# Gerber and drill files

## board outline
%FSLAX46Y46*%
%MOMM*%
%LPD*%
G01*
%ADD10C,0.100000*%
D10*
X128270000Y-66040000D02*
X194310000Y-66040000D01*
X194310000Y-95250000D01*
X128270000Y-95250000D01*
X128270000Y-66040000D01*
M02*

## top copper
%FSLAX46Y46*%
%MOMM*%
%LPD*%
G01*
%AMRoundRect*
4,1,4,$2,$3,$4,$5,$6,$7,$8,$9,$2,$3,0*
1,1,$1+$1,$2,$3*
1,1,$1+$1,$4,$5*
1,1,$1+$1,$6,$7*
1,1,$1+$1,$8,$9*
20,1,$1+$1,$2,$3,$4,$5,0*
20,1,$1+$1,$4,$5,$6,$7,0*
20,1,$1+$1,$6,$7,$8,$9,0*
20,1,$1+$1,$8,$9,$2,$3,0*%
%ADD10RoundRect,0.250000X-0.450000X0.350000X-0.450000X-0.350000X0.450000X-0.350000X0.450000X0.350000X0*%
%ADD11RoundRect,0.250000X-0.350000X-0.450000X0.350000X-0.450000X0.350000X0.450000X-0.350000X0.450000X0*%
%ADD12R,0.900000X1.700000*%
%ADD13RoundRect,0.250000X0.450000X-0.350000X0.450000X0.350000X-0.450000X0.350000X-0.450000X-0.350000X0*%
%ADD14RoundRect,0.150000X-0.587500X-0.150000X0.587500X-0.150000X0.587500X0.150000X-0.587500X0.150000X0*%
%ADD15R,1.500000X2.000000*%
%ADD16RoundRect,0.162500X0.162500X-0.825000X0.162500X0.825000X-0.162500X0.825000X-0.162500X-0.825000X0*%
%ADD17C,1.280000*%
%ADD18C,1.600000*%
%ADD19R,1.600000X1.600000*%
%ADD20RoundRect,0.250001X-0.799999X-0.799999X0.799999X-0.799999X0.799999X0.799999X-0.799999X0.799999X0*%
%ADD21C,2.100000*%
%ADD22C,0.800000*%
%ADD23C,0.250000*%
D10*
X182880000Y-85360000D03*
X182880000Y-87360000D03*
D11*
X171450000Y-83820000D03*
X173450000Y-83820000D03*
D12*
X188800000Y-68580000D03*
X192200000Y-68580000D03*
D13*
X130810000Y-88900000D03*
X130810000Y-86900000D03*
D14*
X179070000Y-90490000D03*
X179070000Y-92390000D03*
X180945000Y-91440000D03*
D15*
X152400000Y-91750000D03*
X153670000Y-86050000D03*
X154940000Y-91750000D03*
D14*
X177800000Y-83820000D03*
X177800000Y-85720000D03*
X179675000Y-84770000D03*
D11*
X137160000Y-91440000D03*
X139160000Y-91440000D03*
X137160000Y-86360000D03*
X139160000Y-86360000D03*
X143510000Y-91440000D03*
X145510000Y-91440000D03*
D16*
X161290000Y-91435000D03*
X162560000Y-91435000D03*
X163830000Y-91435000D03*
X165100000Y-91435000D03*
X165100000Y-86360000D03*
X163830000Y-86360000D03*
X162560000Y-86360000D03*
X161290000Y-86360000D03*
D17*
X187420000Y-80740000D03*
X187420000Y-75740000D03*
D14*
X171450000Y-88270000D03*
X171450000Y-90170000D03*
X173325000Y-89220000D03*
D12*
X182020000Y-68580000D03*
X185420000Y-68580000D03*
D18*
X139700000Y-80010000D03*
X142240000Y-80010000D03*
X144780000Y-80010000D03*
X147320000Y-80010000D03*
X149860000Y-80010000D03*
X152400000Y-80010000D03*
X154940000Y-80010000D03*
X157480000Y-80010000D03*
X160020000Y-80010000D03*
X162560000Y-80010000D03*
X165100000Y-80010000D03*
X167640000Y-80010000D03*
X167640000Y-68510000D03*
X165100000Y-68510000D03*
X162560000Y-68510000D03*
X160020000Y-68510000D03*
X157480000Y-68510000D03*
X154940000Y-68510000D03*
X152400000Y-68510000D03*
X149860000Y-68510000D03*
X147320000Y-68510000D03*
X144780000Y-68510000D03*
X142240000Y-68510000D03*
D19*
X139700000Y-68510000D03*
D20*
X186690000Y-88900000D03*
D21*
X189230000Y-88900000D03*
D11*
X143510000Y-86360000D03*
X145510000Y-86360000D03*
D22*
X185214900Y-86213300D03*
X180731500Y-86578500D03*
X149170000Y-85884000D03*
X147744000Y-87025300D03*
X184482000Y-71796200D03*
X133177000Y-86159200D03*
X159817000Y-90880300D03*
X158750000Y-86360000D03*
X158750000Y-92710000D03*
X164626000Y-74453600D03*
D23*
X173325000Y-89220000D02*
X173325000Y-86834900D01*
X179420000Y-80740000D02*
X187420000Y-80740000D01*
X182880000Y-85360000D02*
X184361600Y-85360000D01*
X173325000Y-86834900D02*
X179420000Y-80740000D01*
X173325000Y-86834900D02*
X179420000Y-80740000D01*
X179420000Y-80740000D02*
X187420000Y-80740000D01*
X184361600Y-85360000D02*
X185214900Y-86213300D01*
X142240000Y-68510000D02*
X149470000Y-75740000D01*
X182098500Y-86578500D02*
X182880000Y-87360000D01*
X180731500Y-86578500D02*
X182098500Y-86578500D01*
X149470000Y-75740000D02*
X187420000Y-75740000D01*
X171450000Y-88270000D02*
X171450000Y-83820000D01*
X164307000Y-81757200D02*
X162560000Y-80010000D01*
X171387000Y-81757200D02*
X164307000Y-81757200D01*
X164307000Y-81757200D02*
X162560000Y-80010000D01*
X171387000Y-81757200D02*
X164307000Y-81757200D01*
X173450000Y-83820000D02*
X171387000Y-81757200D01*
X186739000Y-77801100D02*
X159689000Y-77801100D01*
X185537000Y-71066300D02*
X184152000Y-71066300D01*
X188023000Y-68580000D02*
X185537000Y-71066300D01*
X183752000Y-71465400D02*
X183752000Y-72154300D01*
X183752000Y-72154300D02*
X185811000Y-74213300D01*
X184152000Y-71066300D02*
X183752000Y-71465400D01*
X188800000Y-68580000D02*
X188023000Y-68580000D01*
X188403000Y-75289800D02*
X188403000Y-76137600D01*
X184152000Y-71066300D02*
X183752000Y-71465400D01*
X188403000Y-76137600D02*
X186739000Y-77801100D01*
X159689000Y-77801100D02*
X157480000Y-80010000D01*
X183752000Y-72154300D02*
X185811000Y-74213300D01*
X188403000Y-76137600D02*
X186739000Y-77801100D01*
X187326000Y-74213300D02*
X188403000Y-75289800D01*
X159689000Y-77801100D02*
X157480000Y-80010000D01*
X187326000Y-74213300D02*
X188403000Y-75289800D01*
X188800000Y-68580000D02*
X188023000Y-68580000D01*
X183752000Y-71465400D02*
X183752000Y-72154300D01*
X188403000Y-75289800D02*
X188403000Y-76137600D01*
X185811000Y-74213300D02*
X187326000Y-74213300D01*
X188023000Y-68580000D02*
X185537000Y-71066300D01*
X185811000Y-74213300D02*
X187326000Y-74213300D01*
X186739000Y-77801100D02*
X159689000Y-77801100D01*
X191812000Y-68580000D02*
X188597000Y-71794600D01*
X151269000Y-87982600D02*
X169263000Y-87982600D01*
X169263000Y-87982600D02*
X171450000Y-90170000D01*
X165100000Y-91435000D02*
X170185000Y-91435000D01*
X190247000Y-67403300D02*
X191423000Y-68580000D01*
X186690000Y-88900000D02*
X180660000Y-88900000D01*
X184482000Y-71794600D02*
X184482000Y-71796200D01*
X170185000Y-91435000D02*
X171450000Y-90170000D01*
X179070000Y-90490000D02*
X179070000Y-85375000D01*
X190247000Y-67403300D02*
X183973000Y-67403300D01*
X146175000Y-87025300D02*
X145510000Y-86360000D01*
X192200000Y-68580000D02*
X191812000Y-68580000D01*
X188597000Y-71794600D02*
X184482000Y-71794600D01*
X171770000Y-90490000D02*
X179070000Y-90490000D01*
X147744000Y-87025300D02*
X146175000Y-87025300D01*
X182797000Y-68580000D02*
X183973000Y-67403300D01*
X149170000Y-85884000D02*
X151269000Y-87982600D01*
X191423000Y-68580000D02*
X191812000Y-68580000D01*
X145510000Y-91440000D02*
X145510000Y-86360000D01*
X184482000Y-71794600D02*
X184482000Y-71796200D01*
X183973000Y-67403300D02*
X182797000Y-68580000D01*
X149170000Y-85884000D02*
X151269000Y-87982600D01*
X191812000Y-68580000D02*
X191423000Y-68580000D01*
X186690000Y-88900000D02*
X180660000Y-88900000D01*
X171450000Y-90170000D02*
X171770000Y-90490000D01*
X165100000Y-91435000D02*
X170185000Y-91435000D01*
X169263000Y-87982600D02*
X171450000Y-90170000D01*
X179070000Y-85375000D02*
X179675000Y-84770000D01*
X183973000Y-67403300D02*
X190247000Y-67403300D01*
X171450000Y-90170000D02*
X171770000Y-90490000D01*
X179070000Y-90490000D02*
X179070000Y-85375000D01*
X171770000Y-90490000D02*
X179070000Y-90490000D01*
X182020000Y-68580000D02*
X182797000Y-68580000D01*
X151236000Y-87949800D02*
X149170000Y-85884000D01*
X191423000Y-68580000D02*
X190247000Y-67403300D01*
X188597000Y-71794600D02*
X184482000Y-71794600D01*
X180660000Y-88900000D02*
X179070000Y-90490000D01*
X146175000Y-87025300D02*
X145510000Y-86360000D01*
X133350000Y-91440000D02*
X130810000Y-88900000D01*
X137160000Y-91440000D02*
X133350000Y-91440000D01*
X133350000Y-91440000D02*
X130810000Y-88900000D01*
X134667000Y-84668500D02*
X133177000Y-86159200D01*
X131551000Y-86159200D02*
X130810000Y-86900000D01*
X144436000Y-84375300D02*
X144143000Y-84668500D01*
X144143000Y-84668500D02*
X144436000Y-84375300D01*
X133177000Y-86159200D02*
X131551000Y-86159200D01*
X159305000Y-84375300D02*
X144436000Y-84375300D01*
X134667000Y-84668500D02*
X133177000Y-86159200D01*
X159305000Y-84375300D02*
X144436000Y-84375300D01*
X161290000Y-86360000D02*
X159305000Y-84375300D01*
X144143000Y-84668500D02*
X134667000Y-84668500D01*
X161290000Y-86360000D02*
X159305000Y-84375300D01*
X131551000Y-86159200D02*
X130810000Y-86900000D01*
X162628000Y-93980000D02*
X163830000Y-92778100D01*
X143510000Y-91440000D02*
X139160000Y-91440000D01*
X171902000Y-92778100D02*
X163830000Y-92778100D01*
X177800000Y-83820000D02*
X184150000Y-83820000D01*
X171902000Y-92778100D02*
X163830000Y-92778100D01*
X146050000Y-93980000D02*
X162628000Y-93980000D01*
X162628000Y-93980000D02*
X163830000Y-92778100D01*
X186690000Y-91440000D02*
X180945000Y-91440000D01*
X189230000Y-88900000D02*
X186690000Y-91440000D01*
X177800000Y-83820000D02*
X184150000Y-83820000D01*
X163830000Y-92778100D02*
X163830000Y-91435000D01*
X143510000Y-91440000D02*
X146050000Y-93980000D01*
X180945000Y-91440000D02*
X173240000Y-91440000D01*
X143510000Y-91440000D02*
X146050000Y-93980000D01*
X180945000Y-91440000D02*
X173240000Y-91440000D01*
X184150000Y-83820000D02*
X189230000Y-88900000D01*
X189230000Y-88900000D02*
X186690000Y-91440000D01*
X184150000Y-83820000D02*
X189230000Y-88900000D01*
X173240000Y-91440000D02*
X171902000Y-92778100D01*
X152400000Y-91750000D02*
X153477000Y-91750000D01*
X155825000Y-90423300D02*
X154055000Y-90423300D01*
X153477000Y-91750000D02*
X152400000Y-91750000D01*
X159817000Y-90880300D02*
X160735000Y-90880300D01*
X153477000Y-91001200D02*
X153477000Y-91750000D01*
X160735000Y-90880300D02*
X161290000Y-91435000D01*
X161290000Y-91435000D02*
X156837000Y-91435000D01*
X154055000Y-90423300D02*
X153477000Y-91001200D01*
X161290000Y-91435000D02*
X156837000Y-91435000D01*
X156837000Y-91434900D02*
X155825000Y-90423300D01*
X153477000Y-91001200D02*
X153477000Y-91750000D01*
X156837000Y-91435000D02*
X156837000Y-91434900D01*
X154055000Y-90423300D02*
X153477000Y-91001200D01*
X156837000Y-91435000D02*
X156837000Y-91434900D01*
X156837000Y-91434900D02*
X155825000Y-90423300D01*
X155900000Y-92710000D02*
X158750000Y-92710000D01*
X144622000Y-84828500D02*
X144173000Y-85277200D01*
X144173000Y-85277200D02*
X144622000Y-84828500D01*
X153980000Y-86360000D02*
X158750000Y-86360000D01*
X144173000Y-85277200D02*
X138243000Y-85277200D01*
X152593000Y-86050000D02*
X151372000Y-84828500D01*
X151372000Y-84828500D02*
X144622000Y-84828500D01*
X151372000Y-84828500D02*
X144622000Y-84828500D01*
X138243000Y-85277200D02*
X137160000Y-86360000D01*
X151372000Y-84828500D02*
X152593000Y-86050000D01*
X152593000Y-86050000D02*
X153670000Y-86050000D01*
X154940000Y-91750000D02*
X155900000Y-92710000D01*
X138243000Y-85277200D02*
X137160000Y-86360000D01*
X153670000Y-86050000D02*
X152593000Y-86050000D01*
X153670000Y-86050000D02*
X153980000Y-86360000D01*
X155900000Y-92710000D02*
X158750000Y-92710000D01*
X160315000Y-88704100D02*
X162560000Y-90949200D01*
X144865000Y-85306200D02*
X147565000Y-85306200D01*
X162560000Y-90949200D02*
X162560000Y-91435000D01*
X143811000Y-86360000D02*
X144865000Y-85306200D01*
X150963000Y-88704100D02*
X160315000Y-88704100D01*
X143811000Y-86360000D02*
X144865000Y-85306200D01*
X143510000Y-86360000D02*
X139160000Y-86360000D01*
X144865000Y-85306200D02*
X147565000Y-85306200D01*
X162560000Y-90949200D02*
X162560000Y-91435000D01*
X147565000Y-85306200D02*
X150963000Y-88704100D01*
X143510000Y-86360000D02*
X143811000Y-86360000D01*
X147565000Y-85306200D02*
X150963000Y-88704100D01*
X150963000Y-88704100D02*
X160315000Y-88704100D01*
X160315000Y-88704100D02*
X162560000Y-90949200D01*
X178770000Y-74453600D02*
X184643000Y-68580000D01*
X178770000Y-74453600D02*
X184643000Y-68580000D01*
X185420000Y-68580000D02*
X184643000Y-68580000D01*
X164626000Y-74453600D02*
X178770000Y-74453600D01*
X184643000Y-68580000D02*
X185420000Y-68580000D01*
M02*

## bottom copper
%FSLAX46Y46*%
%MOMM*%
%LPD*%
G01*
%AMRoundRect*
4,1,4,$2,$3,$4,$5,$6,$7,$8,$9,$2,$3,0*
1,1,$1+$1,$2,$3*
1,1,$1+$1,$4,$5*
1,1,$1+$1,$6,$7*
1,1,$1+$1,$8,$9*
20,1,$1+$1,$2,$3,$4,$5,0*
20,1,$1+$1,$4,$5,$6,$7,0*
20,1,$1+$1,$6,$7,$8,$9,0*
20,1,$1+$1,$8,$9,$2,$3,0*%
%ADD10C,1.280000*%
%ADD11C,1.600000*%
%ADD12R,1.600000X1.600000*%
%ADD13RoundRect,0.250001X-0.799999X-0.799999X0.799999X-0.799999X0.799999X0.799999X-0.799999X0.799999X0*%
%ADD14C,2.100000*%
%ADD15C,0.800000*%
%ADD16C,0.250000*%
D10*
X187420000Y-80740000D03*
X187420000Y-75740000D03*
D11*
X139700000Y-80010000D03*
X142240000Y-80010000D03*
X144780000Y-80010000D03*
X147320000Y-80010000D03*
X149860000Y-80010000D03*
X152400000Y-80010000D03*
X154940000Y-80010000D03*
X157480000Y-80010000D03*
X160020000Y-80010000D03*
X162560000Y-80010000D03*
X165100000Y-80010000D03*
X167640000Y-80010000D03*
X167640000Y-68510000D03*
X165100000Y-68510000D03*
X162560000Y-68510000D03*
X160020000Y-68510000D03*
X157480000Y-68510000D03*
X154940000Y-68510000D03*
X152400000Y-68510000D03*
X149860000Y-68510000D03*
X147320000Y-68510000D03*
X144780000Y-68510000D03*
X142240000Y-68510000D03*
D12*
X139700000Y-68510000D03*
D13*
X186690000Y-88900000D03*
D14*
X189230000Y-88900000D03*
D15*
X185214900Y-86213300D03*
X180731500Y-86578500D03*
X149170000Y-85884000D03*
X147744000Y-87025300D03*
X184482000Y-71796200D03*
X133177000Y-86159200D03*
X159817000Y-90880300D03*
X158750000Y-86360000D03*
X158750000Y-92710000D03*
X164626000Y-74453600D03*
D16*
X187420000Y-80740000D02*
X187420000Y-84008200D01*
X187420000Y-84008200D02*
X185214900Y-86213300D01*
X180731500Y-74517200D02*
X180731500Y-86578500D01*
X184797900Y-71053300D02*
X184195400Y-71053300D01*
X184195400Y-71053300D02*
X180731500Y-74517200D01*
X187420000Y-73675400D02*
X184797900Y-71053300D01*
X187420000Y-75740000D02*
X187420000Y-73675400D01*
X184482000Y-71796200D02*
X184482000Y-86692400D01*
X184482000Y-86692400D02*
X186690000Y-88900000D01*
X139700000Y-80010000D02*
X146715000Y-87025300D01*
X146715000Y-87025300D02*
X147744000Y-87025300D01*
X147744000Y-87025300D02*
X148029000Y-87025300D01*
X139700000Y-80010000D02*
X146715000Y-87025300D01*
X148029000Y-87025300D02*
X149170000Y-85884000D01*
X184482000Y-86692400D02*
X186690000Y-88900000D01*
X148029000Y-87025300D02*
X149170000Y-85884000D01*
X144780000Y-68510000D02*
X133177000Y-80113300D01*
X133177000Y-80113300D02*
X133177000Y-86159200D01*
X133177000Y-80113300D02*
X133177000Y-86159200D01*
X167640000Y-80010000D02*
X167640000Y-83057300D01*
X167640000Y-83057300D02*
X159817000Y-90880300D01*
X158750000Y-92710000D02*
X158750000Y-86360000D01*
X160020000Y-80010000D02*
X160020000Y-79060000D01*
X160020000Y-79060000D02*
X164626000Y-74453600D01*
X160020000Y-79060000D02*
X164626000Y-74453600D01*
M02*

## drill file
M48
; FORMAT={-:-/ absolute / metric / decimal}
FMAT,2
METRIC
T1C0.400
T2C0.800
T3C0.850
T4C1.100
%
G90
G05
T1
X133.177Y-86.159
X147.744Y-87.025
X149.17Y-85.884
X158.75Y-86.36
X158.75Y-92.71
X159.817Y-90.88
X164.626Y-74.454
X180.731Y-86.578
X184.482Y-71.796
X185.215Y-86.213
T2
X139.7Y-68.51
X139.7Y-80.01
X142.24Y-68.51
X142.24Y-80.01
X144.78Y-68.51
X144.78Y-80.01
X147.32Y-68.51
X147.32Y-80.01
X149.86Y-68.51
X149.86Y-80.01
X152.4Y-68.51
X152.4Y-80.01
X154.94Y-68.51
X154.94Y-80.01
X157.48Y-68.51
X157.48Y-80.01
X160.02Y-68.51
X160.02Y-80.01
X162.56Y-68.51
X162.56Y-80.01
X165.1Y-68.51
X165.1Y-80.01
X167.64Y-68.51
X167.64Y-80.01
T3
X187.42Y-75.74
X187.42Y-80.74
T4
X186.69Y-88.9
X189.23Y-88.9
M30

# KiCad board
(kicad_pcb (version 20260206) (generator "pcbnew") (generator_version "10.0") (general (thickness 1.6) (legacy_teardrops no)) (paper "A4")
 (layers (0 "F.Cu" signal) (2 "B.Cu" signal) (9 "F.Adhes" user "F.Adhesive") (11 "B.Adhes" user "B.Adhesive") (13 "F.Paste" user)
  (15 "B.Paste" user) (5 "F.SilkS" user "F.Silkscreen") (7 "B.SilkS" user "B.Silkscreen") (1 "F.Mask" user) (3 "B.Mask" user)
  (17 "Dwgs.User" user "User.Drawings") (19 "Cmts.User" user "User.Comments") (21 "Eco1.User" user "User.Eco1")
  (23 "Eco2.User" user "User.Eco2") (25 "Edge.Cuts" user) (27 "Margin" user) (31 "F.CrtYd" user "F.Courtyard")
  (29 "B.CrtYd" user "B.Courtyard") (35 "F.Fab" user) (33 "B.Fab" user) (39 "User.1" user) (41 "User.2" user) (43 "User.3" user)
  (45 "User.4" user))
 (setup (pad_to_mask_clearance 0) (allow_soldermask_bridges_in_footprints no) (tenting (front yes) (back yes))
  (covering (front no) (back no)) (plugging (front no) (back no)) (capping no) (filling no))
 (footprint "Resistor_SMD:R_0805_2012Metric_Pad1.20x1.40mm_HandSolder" (layer "F.Cu") (at 182.88 86.36 -90)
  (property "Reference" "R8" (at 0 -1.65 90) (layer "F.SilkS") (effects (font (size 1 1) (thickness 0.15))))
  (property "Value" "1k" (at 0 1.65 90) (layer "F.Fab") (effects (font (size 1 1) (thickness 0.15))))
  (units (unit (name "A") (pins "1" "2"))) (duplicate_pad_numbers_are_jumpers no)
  (pad "1" smd roundrect (at -1 0 270) (size 1.2 1.4) (layers "F.Cu" "F.Mask" "F.Paste") (roundrect_rratio 0.208333) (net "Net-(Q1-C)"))
  (pad "2" smd roundrect (at 1 0 270) (size 1.2 1.4) (layers "F.Cu" "F.Mask" "F.Paste") (roundrect_rratio 0.208333) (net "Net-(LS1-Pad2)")))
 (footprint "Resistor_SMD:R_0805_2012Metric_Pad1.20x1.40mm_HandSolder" (layer "F.Cu") (at 172.45 83.82)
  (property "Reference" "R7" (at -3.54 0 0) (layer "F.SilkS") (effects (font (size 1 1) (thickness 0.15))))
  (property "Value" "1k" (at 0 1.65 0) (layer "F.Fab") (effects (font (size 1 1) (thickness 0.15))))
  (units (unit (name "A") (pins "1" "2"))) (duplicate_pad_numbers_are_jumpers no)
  (pad "1" smd roundrect (at -1 0) (size 1.2 1.4) (layers "F.Cu" "F.Mask" "F.Paste") (roundrect_rratio 0.208333) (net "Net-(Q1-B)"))
  (pad "2" smd roundrect (at 1 0) (size 1.2 1.4) (layers "F.Cu" "F.Mask" "F.Paste") (roundrect_rratio 0.208333) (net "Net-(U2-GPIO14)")))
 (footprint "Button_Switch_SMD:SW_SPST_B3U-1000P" (layer "F.Cu") (at 190.5 68.58)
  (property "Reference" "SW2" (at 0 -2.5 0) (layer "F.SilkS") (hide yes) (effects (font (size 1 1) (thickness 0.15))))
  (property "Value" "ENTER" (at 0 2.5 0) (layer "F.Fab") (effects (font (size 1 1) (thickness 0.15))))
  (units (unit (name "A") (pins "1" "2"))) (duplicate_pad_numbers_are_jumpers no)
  (pad "1" smd rect (at -1.7 0) (size 0.9 1.7) (layers "F.Cu" "F.Mask" "F.Paste") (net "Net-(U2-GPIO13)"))
  (pad "2" smd rect (at 1.7 0) (size 0.9 1.7) (layers "F.Cu" "F.Mask" "F.Paste") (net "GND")))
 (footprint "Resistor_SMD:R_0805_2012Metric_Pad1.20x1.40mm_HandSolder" (layer "F.Cu") (at 130.81 87.9 90)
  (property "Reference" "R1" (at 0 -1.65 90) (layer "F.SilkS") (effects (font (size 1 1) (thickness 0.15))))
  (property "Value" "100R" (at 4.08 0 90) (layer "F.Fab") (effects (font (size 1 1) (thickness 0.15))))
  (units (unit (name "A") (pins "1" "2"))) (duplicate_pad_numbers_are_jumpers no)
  (pad "1" smd roundrect (at -1 0 90) (size 1.2 1.4) (layers "F.Cu" "F.Mask" "F.Paste") (roundrect_rratio 0.208333) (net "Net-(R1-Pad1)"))
  (pad "2" smd roundrect (at 1 0 90) (size 1.2 1.4) (layers "F.Cu" "F.Mask" "F.Paste") (roundrect_rratio 0.208333) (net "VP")))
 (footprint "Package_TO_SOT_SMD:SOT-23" (layer "F.Cu") (at 180.0075 91.44)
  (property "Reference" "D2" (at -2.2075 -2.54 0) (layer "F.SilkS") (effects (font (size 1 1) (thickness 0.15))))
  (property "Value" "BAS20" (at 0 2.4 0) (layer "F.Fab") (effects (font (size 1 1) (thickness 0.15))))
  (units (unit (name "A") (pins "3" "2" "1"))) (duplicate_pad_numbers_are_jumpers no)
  (pad "1" smd roundrect (at -0.9375 -0.95) (size 1.475 0.6) (layers "F.Cu" "F.Mask" "F.Paste") (roundrect_rratio 0.25) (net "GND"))
  (pad "2" smd roundrect (at -0.9375 0.95) (size 1.475 0.6) (layers "F.Cu" "F.Mask" "F.Paste") (roundrect_rratio 0.25)
   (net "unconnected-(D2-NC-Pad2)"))
  (pad "3" smd roundrect (at 0.9375 0) (size 1.475 0.6) (layers "F.Cu" "F.Mask" "F.Paste") (roundrect_rratio 0.25) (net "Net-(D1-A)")))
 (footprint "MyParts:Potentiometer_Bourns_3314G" (layer "F.Cu") (at 153.67 88.9)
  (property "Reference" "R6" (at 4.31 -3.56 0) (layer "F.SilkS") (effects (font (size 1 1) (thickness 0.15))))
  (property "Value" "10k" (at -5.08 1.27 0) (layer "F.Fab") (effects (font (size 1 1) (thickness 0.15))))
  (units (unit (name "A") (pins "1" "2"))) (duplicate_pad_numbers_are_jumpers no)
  (pad "1" smd rect (at -1.27 2.85) (size 1.5 2) (layers "F.Cu" "F.Mask" "F.Paste") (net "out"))
  (pad "2" smd rect (at 0 -2.85) (size 1.5 2) (layers "F.Cu" "F.Mask" "F.Paste") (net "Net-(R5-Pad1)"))
  (pad "3" smd rect (at 1.27 2.85) (size 1.5 2) (layers "F.Cu" "F.Mask" "F.Paste")))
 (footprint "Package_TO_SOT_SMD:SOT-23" (layer "F.Cu") (at 178.7375 84.77)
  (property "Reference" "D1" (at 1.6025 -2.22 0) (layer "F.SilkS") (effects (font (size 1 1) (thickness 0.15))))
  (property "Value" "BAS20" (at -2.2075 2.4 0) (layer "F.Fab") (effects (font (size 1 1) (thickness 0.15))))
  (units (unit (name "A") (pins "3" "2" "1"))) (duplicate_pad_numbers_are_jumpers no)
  (pad "1" smd roundrect (at -0.9375 -0.95) (size 1.475 0.6) (layers "F.Cu" "F.Mask" "F.Paste") (roundrect_rratio 0.25) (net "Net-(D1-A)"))
  (pad "2" smd roundrect (at -0.9375 0.95) (size 1.475 0.6) (layers "F.Cu" "F.Mask" "F.Paste") (roundrect_rratio 0.25)
   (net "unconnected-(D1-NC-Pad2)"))
  (pad "3" smd roundrect (at 0.9375 0) (size 1.475 0.6) (layers "F.Cu" "F.Mask" "F.Paste") (roundrect_rratio 0.25) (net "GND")))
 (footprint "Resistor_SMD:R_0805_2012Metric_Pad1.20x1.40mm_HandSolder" (layer "F.Cu") (at 138.16 91.44)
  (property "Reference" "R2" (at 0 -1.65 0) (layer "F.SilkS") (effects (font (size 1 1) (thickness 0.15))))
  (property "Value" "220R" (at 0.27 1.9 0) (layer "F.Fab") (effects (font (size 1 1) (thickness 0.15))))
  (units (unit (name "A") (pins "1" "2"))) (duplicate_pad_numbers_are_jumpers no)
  (pad "1" smd roundrect (at -1 0) (size 1.2 1.4) (layers "F.Cu" "F.Mask" "F.Paste") (roundrect_rratio 0.208333) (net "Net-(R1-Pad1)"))
  (pad "2" smd roundrect (at 1 0) (size 1.2 1.4) (layers "F.Cu" "F.Mask" "F.Paste") (roundrect_rratio 0.208333) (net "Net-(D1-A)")))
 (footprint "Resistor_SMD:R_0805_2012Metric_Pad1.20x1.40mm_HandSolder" (layer "F.Cu") (at 138.16 86.36)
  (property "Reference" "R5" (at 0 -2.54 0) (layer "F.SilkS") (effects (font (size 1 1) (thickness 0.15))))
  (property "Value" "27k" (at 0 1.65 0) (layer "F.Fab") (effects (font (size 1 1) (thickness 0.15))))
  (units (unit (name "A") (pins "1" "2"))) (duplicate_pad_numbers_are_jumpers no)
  (pad "1" smd roundrect (at -1 0) (size 1.2 1.4) (layers "F.Cu" "F.Mask" "F.Paste") (roundrect_rratio 0.208333) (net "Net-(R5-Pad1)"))
  (pad "2" smd roundrect (at 1 0) (size 1.2 1.4) (layers "F.Cu" "F.Mask" "F.Paste") (roundrect_rratio 0.208333) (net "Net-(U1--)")))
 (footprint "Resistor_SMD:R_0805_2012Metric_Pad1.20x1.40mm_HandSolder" (layer "F.Cu") (at 144.51 91.44)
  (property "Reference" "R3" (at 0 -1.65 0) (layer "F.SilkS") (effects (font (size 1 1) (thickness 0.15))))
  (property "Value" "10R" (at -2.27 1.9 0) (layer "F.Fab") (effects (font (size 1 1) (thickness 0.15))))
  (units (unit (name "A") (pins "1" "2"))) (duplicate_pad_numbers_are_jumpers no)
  (pad "1" smd roundrect (at -1 0) (size 1.2 1.4) (layers "F.Cu" "F.Mask" "F.Paste") (roundrect_rratio 0.208333) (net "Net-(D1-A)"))
  (pad "2" smd roundrect (at 1 0) (size 1.2 1.4) (layers "F.Cu" "F.Mask" "F.Paste") (roundrect_rratio 0.208333) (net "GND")))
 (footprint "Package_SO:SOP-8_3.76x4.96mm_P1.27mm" (layer "F.Cu") (at 163.195 88.8975 90)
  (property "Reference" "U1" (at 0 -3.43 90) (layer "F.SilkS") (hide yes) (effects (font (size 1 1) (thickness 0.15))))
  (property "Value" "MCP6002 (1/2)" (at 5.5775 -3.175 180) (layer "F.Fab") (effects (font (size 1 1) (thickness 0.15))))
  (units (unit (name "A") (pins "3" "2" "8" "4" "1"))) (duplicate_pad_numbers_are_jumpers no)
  (pad "1" smd roundrect (at -2.5375 -1.905 90) (size 1.975 0.65) (layers "F.Cu" "F.Mask" "F.Paste") (roundrect_rratio 0.25) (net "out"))
  (pad "2" smd roundrect (at -2.5375 -0.635 90) (size 1.975 0.65) (layers "F.Cu" "F.Mask" "F.Paste") (roundrect_rratio 0.25)
   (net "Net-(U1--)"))
  (pad "3" smd roundrect (at -2.5375 0.635 90) (size 1.975 0.65) (layers "F.Cu" "F.Mask" "F.Paste") (roundrect_rratio 0.25)
   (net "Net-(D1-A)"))
  (pad "4" smd roundrect (at -2.5375 1.905 90) (size 1.975 0.65) (layers "F.Cu" "F.Mask" "F.Paste") (roundrect_rratio 0.25) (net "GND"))
  (pad "5" smd roundrect (at 2.5375 1.905 90) (size 1.975 0.65) (layers "F.Cu" "F.Mask" "F.Paste") (roundrect_rratio 0.25))
  (pad "6" smd roundrect (at 2.5375 0.635 90) (size 1.975 0.65) (layers "F.Cu" "F.Mask" "F.Paste") (roundrect_rratio 0.25))
  (pad "7" smd roundrect (at 2.5375 -0.635 90) (size 1.975 0.65) (layers "F.Cu" "F.Mask" "F.Paste") (roundrect_rratio 0.25))
  (pad "8" smd roundrect (at 2.5375 -1.905 90) (size 1.975 0.65) (layers "F.Cu" "F.Mask" "F.Paste") (roundrect_rratio 0.25) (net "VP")))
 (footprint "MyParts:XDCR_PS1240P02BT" (layer "F.Cu") (at 187.42 78.24 90)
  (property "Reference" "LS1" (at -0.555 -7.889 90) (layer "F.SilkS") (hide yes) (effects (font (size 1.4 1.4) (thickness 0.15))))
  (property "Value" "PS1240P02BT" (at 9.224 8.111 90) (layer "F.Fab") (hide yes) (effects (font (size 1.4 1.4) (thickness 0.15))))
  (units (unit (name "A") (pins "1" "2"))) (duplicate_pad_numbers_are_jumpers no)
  (pad "1" thru_hole circle (at -2.5 0 90) (size 1.28 1.28) (drill 0.85) (layers "*.Cu" "*.Mask") (remove_unused_layers no)
   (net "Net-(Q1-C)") (solder_mask_margin 0.102))
  (pad "2" thru_hole circle (at 2.5 0 90) (size 1.28 1.28) (drill 0.85) (layers "*.Cu" "*.Mask") (remove_unused_layers no)
   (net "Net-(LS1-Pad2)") (solder_mask_margin 0.102)))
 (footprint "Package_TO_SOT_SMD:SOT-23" (layer "F.Cu") (at 172.3875 89.22)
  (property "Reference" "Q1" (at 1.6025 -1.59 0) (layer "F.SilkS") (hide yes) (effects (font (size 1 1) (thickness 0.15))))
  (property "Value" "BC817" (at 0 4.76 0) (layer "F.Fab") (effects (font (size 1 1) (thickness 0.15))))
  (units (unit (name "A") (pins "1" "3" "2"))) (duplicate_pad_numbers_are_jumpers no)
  (pad "1" smd roundrect (at -0.9375 -0.95) (size 1.475 0.6) (layers "F.Cu" "F.Mask" "F.Paste") (roundrect_rratio 0.25) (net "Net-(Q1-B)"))
  (pad "2" smd roundrect (at -0.9375 0.95) (size 1.475 0.6) (layers "F.Cu" "F.Mask" "F.Paste") (roundrect_rratio 0.25) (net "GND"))
  (pad "3" smd roundrect (at 0.9375 0) (size 1.475 0.6) (layers "F.Cu" "F.Mask" "F.Paste") (roundrect_rratio 0.25) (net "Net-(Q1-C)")))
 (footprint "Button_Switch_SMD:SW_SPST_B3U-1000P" (layer "F.Cu") (at 183.72 68.58)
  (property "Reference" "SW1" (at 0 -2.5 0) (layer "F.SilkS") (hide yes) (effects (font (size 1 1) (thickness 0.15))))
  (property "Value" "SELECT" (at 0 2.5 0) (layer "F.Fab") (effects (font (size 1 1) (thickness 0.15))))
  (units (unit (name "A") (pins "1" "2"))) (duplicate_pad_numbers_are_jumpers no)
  (pad "1" smd rect (at -1.7 0) (size 0.9 1.7) (layers "F.Cu" "F.Mask" "F.Paste") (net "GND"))
  (pad "2" smd rect (at 1.7 0) (size 0.9 1.7) (layers "F.Cu" "F.Mask" "F.Paste") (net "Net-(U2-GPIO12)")))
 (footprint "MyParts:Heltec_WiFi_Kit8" (layer "F.Cu") (at 139.7 68.51)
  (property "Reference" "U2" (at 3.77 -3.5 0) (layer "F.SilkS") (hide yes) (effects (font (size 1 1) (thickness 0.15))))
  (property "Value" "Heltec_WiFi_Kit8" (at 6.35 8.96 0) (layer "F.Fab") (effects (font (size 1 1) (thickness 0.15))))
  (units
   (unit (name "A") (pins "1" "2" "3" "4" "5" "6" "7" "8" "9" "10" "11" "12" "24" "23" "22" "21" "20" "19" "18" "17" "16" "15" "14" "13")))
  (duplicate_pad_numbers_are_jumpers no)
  (pad "1" thru_hole circle (at 0 11.5) (size 1.6 1.6) (drill 0.8) (layers "*.Cu" "*.Mask") (remove_unused_layers no) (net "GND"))
  (pad "2" thru_hole circle (at 2.54 11.5) (size 1.6 1.6) (drill 0.8) (layers "*.Cu" "*.Mask") (remove_unused_layers no)
   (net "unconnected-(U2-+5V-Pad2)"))
  (pad "3" thru_hole circle (at 5.08 11.5) (size 1.6 1.6) (drill 0.8) (layers "*.Cu" "*.Mask") (remove_unused_layers no)
   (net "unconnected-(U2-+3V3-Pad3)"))
  (pad "4" thru_hole circle (at 7.62 11.5) (size 1.6 1.6) (drill 0.8) (layers "*.Cu" "*.Mask") (remove_unused_layers no)
   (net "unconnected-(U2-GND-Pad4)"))
  (pad "5" thru_hole circle (at 10.16 11.5) (size 1.6 1.6) (drill 0.8) (layers "*.Cu" "*.Mask") (remove_unused_layers no)
   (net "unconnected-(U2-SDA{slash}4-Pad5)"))
  (pad "6" thru_hole circle (at 12.7 11.5) (size 1.6 1.6) (drill 0.8) (layers "*.Cu" "*.Mask") (remove_unused_layers no)
   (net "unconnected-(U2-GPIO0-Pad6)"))
  (pad "7" thru_hole circle (at 15.24 11.5) (size 1.6 1.6) (drill 0.8) (layers "*.Cu" "*.Mask") (remove_unused_layers no)
   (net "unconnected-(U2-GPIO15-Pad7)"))
  (pad "8" thru_hole circle (at 17.78 11.5) (size 1.6 1.6) (drill 0.8) (layers "*.Cu" "*.Mask") (remove_unused_layers no)
   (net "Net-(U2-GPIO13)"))
  (pad "9" thru_hole circle (at 20.32 11.5) (size 1.6 1.6) (drill 0.8) (layers "*.Cu" "*.Mask") (remove_unused_layers no)
   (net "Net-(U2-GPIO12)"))
  (pad "10" thru_hole circle (at 22.86 11.5) (size 1.6 1.6) (drill 0.8) (layers "*.Cu" "*.Mask") (remove_unused_layers no)
   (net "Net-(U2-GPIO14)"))
  (pad "11" thru_hole circle (at 25.4 11.5) (size 1.6 1.6) (drill 0.8) (layers "*.Cu" "*.Mask") (remove_unused_layers no)
   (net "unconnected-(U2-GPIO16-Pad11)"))
  (pad "12" thru_hole circle (at 27.94 11.5) (size 1.6 1.6) (drill 0.8) (layers "*.Cu" "*.Mask") (remove_unused_layers no) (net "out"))
  (pad "13" thru_hole circle (at 27.94 0) (size 1.6 1.6) (drill 0.8) (layers "*.Cu" "*.Mask") (remove_unused_layers no)
   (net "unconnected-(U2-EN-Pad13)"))
  (pad "14" thru_hole circle (at 25.4 0) (size 1.6 1.6) (drill 0.8) (layers "*.Cu" "*.Mask") (remove_unused_layers no)
   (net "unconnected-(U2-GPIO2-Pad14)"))
  (pad "15" thru_hole circle (at 22.86 0) (size 1.6 1.6) (drill 0.8) (layers "*.Cu" "*.Mask") (remove_unused_layers no)
   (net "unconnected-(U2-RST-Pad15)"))
  (pad "16" thru_hole circle (at 20.32 0) (size 1.6 1.6) (drill 0.8) (layers "*.Cu" "*.Mask") (remove_unused_layers no)
   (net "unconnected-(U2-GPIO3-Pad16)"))
  (pad "17" thru_hole circle (at 17.78 0) (size 1.6 1.6) (drill 0.8) (layers "*.Cu" "*.Mask") (remove_unused_layers no)
   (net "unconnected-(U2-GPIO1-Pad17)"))
  (pad "18" thru_hole circle (at 15.24 0) (size 1.6 1.6) (drill 0.8) (layers "*.Cu" "*.Mask") (remove_unused_layers no)
   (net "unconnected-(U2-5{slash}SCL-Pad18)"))
  (pad "19" thru_hole circle (at 12.7 0) (size 1.6 1.6) (drill 0.8) (layers "*.Cu" "*.Mask") (remove_unused_layers no)
   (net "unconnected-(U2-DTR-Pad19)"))
  (pad "20" thru_hole circle (at 10.16 0) (size 1.6 1.6) (drill 0.8) (layers "*.Cu" "*.Mask") (remove_unused_layers no)
   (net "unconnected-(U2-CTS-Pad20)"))
  (pad "21" thru_hole circle (at 7.62 0) (size 1.6 1.6) (drill 0.8) (layers "*.Cu" "*.Mask") (remove_unused_layers no)
   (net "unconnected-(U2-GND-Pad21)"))
  (pad "22" thru_hole circle (at 5.08 0) (size 1.6 1.6) (drill 0.8) (layers "*.Cu" "*.Mask") (remove_unused_layers no) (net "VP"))
  (pad "23" thru_hole circle (at 2.54 0) (size 1.6 1.6) (drill 0.8) (layers "*.Cu" "*.Mask") (remove_unused_layers no)
   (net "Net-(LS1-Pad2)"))
  (pad "24" thru_hole rect (at 0 0) (size 1.6 1.6) (drill 0.8) (layers "*.Cu" "*.Mask") (remove_unused_layers no)
   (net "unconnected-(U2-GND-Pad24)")))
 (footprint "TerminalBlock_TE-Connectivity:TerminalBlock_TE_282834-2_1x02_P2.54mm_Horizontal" (layer "F.Cu") (at 186.69 88.9)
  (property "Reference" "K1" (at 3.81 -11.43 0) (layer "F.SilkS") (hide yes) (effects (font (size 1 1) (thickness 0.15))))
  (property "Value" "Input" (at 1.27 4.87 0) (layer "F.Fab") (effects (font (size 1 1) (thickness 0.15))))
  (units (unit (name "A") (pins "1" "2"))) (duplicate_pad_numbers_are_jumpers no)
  (pad "1" thru_hole roundrect (at 0 0) (size 2.1 2.1) (drill 1.1) (layers "*.Cu" "*.Mask") (remove_unused_layers no)
   (roundrect_rratio 0.119048) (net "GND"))
  (pad "2" thru_hole circle (at 2.54 0) (size 2.1 2.1) (drill 1.1) (layers "*.Cu" "*.Mask") (remove_unused_layers no) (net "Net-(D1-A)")))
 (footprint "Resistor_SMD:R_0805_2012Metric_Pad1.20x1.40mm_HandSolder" (layer "F.Cu") (at 144.51 86.36)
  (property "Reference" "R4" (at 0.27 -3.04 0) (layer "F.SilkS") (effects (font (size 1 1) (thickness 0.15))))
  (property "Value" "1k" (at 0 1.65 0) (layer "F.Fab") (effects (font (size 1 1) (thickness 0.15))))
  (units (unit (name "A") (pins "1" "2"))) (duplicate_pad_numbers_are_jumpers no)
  (pad "1" smd roundrect (at -1 0) (size 1.2 1.4) (layers "F.Cu" "F.Mask" "F.Paste") (roundrect_rratio 0.208333) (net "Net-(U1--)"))
  (pad "2" smd roundrect (at 1 0) (size 1.2 1.4) (layers "F.Cu" "F.Mask" "F.Paste") (roundrect_rratio 0.208333) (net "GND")))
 (gr_rect (start 128.27 66.04) (end 194.31 95.25) (stroke (width 0.1) (type default)) (fill no) (layer "Edge.Cuts"))
 (segment (start 173.325 89.22) (end 173.325 86.8349) (width 0.25) (layer "F.Cu") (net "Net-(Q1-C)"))
 (segment (start 179.42 80.74) (end 187.42 80.74) (width 0.25) (layer "F.Cu") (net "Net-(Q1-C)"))
 (segment (start 182.88 85.36) (end 184.3616 85.36) (width 0.25) (layer "F.Cu") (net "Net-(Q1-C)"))
 (segment (start 173.325 86.8349) (end 179.42 80.74) (width 0.25) (layer "F.Cu") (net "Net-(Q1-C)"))
 (segment (start 173.325 86.8349) (end 179.42 80.74) (width 0.25) (layer "F.Cu") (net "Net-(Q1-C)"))
 (segment (start 179.42 80.74) (end 187.42 80.74) (width 0.25) (layer "F.Cu") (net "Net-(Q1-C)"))
 (segment (start 184.3616 85.36) (end 185.2149 86.2133) (width 0.25) (layer "F.Cu") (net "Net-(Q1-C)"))
 (via (at 185.2149 86.2133) (size 0.8) (drill 0.4) (layers "F.Cu" "B.Cu") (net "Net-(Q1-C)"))
 (segment (start 187.42 80.74) (end 187.42 84.0082) (width 0.25) (layer "B.Cu") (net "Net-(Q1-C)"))
 (segment (start 187.42 84.0082) (end 185.2149 86.2133) (width 0.25) (layer "B.Cu") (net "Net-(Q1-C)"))
 (segment (start 142.24 68.51) (end 149.47 75.74) (width 0.25) (layer "F.Cu") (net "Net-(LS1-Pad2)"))
 (segment (start 182.0985 86.5785) (end 182.88 87.36) (width 0.25) (layer "F.Cu") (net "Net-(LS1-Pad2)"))
 (segment (start 180.7315 86.5785) (end 182.0985 86.5785) (width 0.25) (layer "F.Cu") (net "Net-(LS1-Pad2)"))
 (segment (start 149.47 75.74) (end 187.42 75.74) (width 0.25) (layer "F.Cu") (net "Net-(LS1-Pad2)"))
 (via (at 180.7315 86.5785) (size 0.8) (drill 0.4) (layers "F.Cu" "B.Cu") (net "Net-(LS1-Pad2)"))
 (segment (start 180.7315 74.5172) (end 180.7315 86.5785) (width 0.25) (layer "B.Cu") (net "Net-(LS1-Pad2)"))
 (segment (start 184.7979 71.0533) (end 184.1954 71.0533) (width 0.25) (layer "B.Cu") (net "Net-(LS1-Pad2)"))
 (segment (start 184.1954 71.0533) (end 180.7315 74.5172) (width 0.25) (layer "B.Cu") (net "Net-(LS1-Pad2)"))
 (segment (start 187.42 73.6754) (end 184.7979 71.0533) (width 0.25) (layer "B.Cu") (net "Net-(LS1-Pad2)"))
 (segment (start 187.42 75.74) (end 187.42 73.6754) (width 0.25) (layer "B.Cu") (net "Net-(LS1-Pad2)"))
 (segment (start 171.45 88.27) (end 171.45 83.82) (width 0.25) (layer "F.Cu") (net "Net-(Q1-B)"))
 (segment (start 164.307 81.7572) (end 162.56 80.01) (width 0.25) (layer "F.Cu") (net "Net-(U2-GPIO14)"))
 (segment (start 171.387 81.7572) (end 164.307 81.7572) (width 0.25) (layer "F.Cu") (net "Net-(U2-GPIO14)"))
 (segment (start 164.307 81.7572) (end 162.56 80.01) (width 0.25) (layer "F.Cu") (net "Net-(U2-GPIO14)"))
 (segment (start 171.387 81.7572) (end 164.307 81.7572) (width 0.25) (layer "F.Cu") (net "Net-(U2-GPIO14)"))
 (segment (start 173.45 83.82) (end 171.387 81.7572) (width 0.25) (layer "F.Cu") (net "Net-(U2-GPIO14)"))
 (segment (start 186.739 77.8011) (end 159.689 77.8011) (width 0.25) (layer "F.Cu") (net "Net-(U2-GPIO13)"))
 (segment (start 185.537 71.0663) (end 184.152 71.0663) (width 0.25) (layer "F.Cu") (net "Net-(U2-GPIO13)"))
 (segment (start 188.023 68.58) (end 185.537 71.0663) (width 0.25) (layer "F.Cu") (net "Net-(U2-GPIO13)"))
 (segment (start 183.752 71.4654) (end 183.752 72.1543) (width 0.25) (layer "F.Cu") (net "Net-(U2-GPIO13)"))
 (segment (start 183.752 72.1543) (end 185.811 74.2133) (width 0.25) (layer "F.Cu") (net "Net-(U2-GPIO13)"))
 (segment (start 184.152 71.0663) (end 183.752 71.4654) (width 0.25) (layer "F.Cu") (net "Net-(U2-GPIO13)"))
 (segment (start 188.8 68.58) (end 188.023 68.58) (width 0.25) (layer "F.Cu") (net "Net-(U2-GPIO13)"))
 (segment (start 188.403 75.2898) (end 188.403 76.1376) (width 0.25) (layer "F.Cu") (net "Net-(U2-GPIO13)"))
 (segment (start 184.152 71.0663) (end 183.752 71.4654) (width 0.25) (layer "F.Cu") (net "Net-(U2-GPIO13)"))
 (segment (start 188.403 76.1376) (end 186.739 77.8011) (width 0.25) (layer "F.Cu") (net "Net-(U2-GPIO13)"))
 (segment (start 159.689 77.8011) (end 157.48 80.01) (width 0.25) (layer "F.Cu") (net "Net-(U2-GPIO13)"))
 (segment (start 183.752 72.1543) (end 185.811 74.2133) (width 0.25) (layer "F.Cu") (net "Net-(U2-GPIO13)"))
 (segment (start 188.403 76.1376) (end 186.739 77.8011) (width 0.25) (layer "F.Cu") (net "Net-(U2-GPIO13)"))
 (segment (start 187.326 74.2133) (end 188.403 75.2898) (width 0.25) (layer "F.Cu") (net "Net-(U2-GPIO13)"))
 (segment (start 159.689 77.8011) (end 157.48 80.01) (width 0.25) (layer "F.Cu") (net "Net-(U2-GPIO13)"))
 (segment (start 187.326 74.2133) (end 188.403 75.2898) (width 0.25) (layer "F.Cu") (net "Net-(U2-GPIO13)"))
 (segment (start 188.8 68.58) (end 188.023 68.58) (width 0.25) (layer "F.Cu") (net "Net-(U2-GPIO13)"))
 (segment (start 183.752 71.4654) (end 183.752 72.1543) (width 0.25) (layer "F.Cu") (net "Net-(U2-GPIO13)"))
 (segment (start 188.403 75.2898) (end 188.403 76.1376) (width 0.25) (layer "F.Cu") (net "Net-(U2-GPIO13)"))
 (segment (start 185.811 74.2133) (end 187.326 74.2133) (width 0.25) (layer "F.Cu") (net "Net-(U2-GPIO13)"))
 (segment (start 188.023 68.58) (end 185.537 71.0663) (width 0.25) (layer "F.Cu") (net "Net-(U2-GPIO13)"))
 (segment (start 185.811 74.2133) (end 187.326 74.2133) (width 0.25) (layer "F.Cu") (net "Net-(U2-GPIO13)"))
 (segment (start 186.739 77.8011) (end 159.689 77.8011) (width 0.25) (layer "F.Cu") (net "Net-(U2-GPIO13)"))
 (segment (start 191.812 68.58) (end 188.597 71.7946) (width 0.25) (layer "F.Cu") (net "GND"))
 (segment (start 151.269 87.9826) (end 169.263 87.9826) (width 0.25) (layer "F.Cu") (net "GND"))
 (segment (start 169.263 87.9826) (end 171.45 90.17) (width 0.25) (layer "F.Cu") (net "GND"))
 (segment (start 165.1 91.435) (end 170.185 91.435) (width 0.25) (layer "F.Cu") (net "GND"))
 (segment (start 190.247 67.4033) (end 191.423 68.58) (width 0.25) (layer "F.Cu") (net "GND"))
 (segment (start 186.69 88.9) (end 180.66 88.9) (width 0.25) (layer "F.Cu") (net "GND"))
 (segment (start 184.482 71.7946) (end 184.482 71.7962) (width 0.25) (layer "F.Cu") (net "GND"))
 (segment (start 170.185 91.435) (end 171.45 90.17) (width 0.25) (layer "F.Cu") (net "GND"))
 (segment (start 179.07 90.49) (end 179.07 85.375) (width 0.25) (layer "F.Cu") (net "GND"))
 (segment (start 190.247 67.4033) (end 183.973 67.4033) (width 0.25) (layer "F.Cu") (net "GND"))
 (segment (start 146.175 87.0253) (end 145.51 86.36) (width 0.25) (layer "F.Cu") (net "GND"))
 (segment (start 192.2 68.58) (end 191.812 68.58) (width 0.25) (layer "F.Cu") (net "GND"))
 (segment (start 188.597 71.7946) (end 184.482 71.7946) (width 0.25) (layer "F.Cu") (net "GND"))
 (segment (start 171.77 90.49) (end 179.07 90.49) (width 0.25) (layer "F.Cu") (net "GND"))
 (segment (start 147.744 87.0253) (end 146.175 87.0253) (width 0.25) (layer "F.Cu") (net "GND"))
 (segment (start 182.797 68.58) (end 183.973 67.4033) (width 0.25) (layer "F.Cu") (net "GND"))
 (segment (start 149.17 85.884) (end 151.269 87.9826) (width 0.25) (layer "F.Cu") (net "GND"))
 (segment (start 191.423 68.58) (end 191.812 68.58) (width 0.25) (layer "F.Cu") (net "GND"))
 (segment (start 145.51 91.44) (end 145.51 86.36) (width 0.25) (layer "F.Cu") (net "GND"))
 (segment (start 184.482 71.7946) (end 184.482 71.7962) (width 0.25) (layer "F.Cu") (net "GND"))
 (segment (start 183.973 67.4033) (end 182.797 68.58) (width 0.25) (layer "F.Cu") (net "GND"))
 (segment (start 149.17 85.884) (end 151.269 87.9826) (width 0.25) (layer "F.Cu") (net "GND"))
 (segment (start 191.812 68.58) (end 191.423 68.58) (width 0.25) (layer "F.Cu") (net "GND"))
 (segment (start 186.69 88.9) (end 180.66 88.9) (width 0.25) (layer "F.Cu") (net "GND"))
 (segment (start 171.45 90.17) (end 171.77 90.49) (width 0.25) (layer "F.Cu") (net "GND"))
 (segment (start 165.1 91.435) (end 170.185 91.435) (width 0.25) (layer "F.Cu") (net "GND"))
 (segment (start 169.263 87.9826) (end 171.45 90.17) (width 0.25) (layer "F.Cu") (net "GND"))
 (segment (start 179.07 85.375) (end 179.675 84.77) (width 0.25) (layer "F.Cu") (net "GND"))
 (segment (start 183.973 67.4033) (end 190.247 67.4033) (width 0.25) (layer "F.Cu") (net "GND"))
 (segment (start 171.45 90.17) (end 171.77 90.49) (width 0.25) (layer "F.Cu") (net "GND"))
 (segment (start 179.07 90.49) (end 179.07 85.375) (width 0.25) (layer "F.Cu") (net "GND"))
 (segment (start 171.77 90.49) (end 179.07 90.49) (width 0.25) (layer "F.Cu") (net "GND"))
 (segment (start 182.02 68.58) (end 182.797 68.58) (width 0.25) (layer "F.Cu") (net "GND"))
 (segment (start 151.236 87.9498) (end 149.17 85.884) (width 0.25) (layer "F.Cu") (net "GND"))
 (segment (start 191.423 68.58) (end 190.247 67.4033) (width 0.25) (layer "F.Cu") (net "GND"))
 (segment (start 188.597 71.7946) (end 184.482 71.7946) (width 0.25) (layer "F.Cu") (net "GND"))
 (segment (start 180.66 88.9) (end 179.07 90.49) (width 0.25) (layer "F.Cu") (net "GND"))
 (segment (start 146.175 87.0253) (end 145.51 86.36) (width 0.25) (layer "F.Cu") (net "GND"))
 (via (at 149.17 85.884) (size 0.8) (drill 0.4) (layers "F.Cu" "B.Cu") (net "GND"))
 (via (at 147.744 87.0253) (size 0.8) (drill 0.4) (layers "F.Cu" "B.Cu") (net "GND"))
 (via (at 184.482 71.7962) (size 0.8) (drill 0.4) (layers "F.Cu" "B.Cu") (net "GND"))
 (segment (start 184.482 71.7962) (end 184.482 86.6924) (width 0.25) (layer "B.Cu") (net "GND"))
 (segment (start 184.482 86.6924) (end 186.69 88.9) (width 0.25) (layer "B.Cu") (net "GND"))
 (segment (start 139.7 80.01) (end 146.715 87.0253) (width 0.25) (layer "B.Cu") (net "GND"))
 (segment (start 146.715 87.0253) (end 147.744 87.0253) (width 0.25) (layer "B.Cu") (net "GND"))
 (segment (start 147.744 87.0253) (end 148.029 87.0253) (width 0.25) (layer "B.Cu") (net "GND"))
 (segment (start 139.7 80.01) (end 146.715 87.0253) (width 0.25) (layer "B.Cu") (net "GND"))
 (segment (start 148.029 87.0253) (end 149.17 85.884) (width 0.25) (layer "B.Cu") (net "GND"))
 (segment (start 184.482 86.6924) (end 186.69 88.9) (width 0.25) (layer "B.Cu") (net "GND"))
 (segment (start 148.029 87.0253) (end 149.17 85.884) (width 0.25) (layer "B.Cu") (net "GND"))
 (segment (start 133.35 91.44) (end 130.81 88.9) (width 0.25) (layer "F.Cu") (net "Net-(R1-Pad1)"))
 (segment (start 137.16 91.44) (end 133.35 91.44) (width 0.25) (layer "F.Cu") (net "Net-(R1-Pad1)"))
 (segment (start 133.35 91.44) (end 130.81 88.9) (width 0.25) (layer "F.Cu") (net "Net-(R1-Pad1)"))
 (segment (start 134.667 84.6685) (end 133.177 86.1592) (width 0.25) (layer "F.Cu") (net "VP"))
 (segment (start 131.551 86.1592) (end 130.81 86.9) (width 0.25) (layer "F.Cu") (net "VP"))
 (segment (start 144.436 84.3753) (end 144.143 84.6685) (width 0.25) (layer "F.Cu") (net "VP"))
 (segment (start 144.143 84.6685) (end 144.436 84.3753) (width 0.25) (layer "F.Cu") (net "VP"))
 (segment (start 133.177 86.1592) (end 131.551 86.1592) (width 0.25) (layer "F.Cu") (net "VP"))
 (segment (start 159.305 84.3753) (end 144.436 84.3753) (width 0.25) (layer "F.Cu") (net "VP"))
 (segment (start 134.667 84.6685) (end 133.177 86.1592) (width 0.25) (layer "F.Cu") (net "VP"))
 (segment (start 159.305 84.3753) (end 144.436 84.3753) (width 0.25) (layer "F.Cu") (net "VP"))
 (segment (start 161.29 86.36) (end 159.305 84.3753) (width 0.25) (layer "F.Cu") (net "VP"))
 (segment (start 144.143 84.6685) (end 134.667 84.6685) (width 0.25) (layer "F.Cu") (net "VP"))
 (segment (start 161.29 86.36) (end 159.305 84.3753) (width 0.25) (layer "F.Cu") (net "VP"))
 (segment (start 131.551 86.1592) (end 130.81 86.9) (width 0.25) (layer "F.Cu") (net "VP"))
 (via (at 133.177 86.1592) (size 0.8) (drill 0.4) (layers "F.Cu" "B.Cu") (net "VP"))
 (segment (start 144.78 68.51) (end 133.177 80.1133) (width 0.25) (layer "B.Cu") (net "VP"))
 (segment (start 133.177 80.1133) (end 133.177 86.1592) (width 0.25) (layer "B.Cu") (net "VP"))
 (segment (start 133.177 80.1133) (end 133.177 86.1592) (width 0.25) (layer "B.Cu") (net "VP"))
 (segment (start 162.628 93.98) (end 163.83 92.7781) (width 0.25) (layer "F.Cu") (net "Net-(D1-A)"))
 (segment (start 143.51 91.44) (end 139.16 91.44) (width 0.25) (layer "F.Cu") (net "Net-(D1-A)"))
 (segment (start 171.902 92.7781) (end 163.83 92.7781) (width 0.25) (layer "F.Cu") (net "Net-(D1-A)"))
 (segment (start 177.8 83.82) (end 184.15 83.82) (width 0.25) (layer "F.Cu") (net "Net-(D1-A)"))
 (segment (start 171.902 92.7781) (end 163.83 92.7781) (width 0.25) (layer "F.Cu") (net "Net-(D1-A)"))
 (segment (start 146.05 93.98) (end 162.628 93.98) (width 0.25) (layer "F.Cu") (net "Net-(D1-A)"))
 (segment (start 162.628 93.98) (end 163.83 92.7781) (width 0.25) (layer "F.Cu") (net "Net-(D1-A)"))
 (segment (start 186.69 91.44) (end 180.945 91.44) (width 0.25) (layer "F.Cu") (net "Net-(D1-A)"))
 (segment (start 189.23 88.9) (end 186.69 91.44) (width 0.25) (layer "F.Cu") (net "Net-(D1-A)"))
 (segment (start 177.8 83.82) (end 184.15 83.82) (width 0.25) (layer "F.Cu") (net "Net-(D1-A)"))
 (segment (start 163.83 92.7781) (end 163.83 91.435) (width 0.25) (layer "F.Cu") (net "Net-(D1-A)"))
 (segment (start 143.51 91.44) (end 146.05 93.98) (width 0.25) (layer "F.Cu") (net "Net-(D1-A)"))
 (segment (start 180.945 91.44) (end 173.24 91.44) (width 0.25) (layer "F.Cu") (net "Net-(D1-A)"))
 (segment (start 143.51 91.44) (end 146.05 93.98) (width 0.25) (layer "F.Cu") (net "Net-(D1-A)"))
 (segment (start 180.945 91.44) (end 173.24 91.44) (width 0.25) (layer "F.Cu") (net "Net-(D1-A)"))
 (segment (start 184.15 83.82) (end 189.23 88.9) (width 0.25) (layer "F.Cu") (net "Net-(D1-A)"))
 (segment (start 189.23 88.9) (end 186.69 91.44) (width 0.25) (layer "F.Cu") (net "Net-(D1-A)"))
 (segment (start 184.15 83.82) (end 189.23 88.9) (width 0.25) (layer "F.Cu") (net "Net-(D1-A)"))
 (segment (start 173.24 91.44) (end 171.902 92.7781) (width 0.25) (layer "F.Cu") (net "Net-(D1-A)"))
 (segment (start 152.4 91.75) (end 153.477 91.75) (width 0.25) (layer "F.Cu") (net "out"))
 (segment (start 155.825 90.4233) (end 154.055 90.4233) (width 0.25) (layer "F.Cu") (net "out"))
 (segment (start 153.477 91.75) (end 152.4 91.75) (width 0.25) (layer "F.Cu") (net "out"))
 (segment (start 159.817 90.8803) (end 160.735 90.8803) (width 0.25) (layer "F.Cu") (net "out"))
 (segment (start 153.477 91.0012) (end 153.477 91.75) (width 0.25) (layer "F.Cu") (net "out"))
 (segment (start 160.735 90.8803) (end 161.29 91.435) (width 0.25) (layer "F.Cu") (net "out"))
 (segment (start 161.29 91.435) (end 156.837 91.435) (width 0.25) (layer "F.Cu") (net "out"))
 (segment (start 154.055 90.4233) (end 153.477 91.0012) (width 0.25) (layer "F.Cu") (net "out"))
 (segment (start 161.29 91.435) (end 156.837 91.435) (width 0.25) (layer "F.Cu") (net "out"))
 (segment (start 156.837 91.4349) (end 155.825 90.4233) (width 0.25) (layer "F.Cu") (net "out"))
 (segment (start 153.477 91.0012) (end 153.477 91.75) (width 0.25) (layer "F.Cu") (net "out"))
 (segment (start 156.837 91.435) (end 156.837 91.4349) (width 0.25) (layer "F.Cu") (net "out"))
 (segment (start 154.055 90.4233) (end 153.477 91.0012) (width 0.25) (layer "F.Cu") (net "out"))
 (segment (start 156.837 91.435) (end 156.837 91.4349) (width 0.25) (layer "F.Cu") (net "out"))
 (segment (start 156.837 91.4349) (end 155.825 90.4233) (width 0.25) (layer "F.Cu") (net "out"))
 (via (at 159.817 90.8803) (size 0.8) (drill 0.4) (layers "F.Cu" "B.Cu") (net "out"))
 (segment (start 167.64 80.01) (end 167.64 83.0573) (width 0.25) (layer "B.Cu") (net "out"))
 (segment (start 167.64 83.0573) (end 159.817 90.8803) (width 0.25) (layer "B.Cu") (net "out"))
 (segment (start 155.9 92.71) (end 158.75 92.71) (width 0.25) (layer "F.Cu") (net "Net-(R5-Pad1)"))
 (segment (start 144.622 84.8285) (end 144.173 85.2772) (width 0.25) (layer "F.Cu") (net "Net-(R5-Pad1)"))
 (segment (start 144.173 85.2772) (end 144.622 84.8285) (width 0.25) (layer "F.Cu") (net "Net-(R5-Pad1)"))
 (segment (start 153.98 86.36) (end 158.75 86.36) (width 0.25) (layer "F.Cu") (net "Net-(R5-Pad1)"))
 (segment (start 144.173 85.2772) (end 138.243 85.2772) (width 0.25) (layer "F.Cu") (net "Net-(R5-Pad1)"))
 (segment (start 152.593 86.05) (end 151.372 84.8285) (width 0.25) (layer "F.Cu") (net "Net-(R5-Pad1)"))
 (segment (start 151.372 84.8285) (end 144.622 84.8285) (width 0.25) (layer "F.Cu") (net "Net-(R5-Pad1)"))
 (segment (start 151.372 84.8285) (end 144.622 84.8285) (width 0.25) (layer "F.Cu") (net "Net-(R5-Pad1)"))
 (segment (start 138.243 85.2772) (end 137.16 86.36) (width 0.25) (layer "F.Cu") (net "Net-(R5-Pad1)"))
 (segment (start 151.372 84.8285) (end 152.593 86.05) (width 0.25) (layer "F.Cu") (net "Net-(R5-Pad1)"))
 (segment (start 152.593 86.05) (end 153.67 86.05) (width 0.25) (layer "F.Cu") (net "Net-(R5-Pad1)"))
 (segment (start 154.94 91.75) (end 155.9 92.71) (width 0.25) (layer "F.Cu") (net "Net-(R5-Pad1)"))
 (segment (start 138.243 85.2772) (end 137.16 86.36) (width 0.25) (layer "F.Cu") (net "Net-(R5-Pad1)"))
 (segment (start 153.67 86.05) (end 152.593 86.05) (width 0.25) (layer "F.Cu") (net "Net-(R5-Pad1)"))
 (segment (start 153.67 86.05) (end 153.98 86.36) (width 0.25) (layer "F.Cu") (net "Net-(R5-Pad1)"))
 (segment (start 155.9 92.71) (end 158.75 92.71) (width 0.25) (layer "F.Cu") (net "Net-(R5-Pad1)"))
 (via (at 158.75 86.36) (size 0.8) (drill 0.4) (layers "F.Cu" "B.Cu") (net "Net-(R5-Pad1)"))
 (via (at 158.75 92.71) (size 0.8) (drill 0.4) (layers "F.Cu" "B.Cu") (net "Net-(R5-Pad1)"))
 (segment (start 158.75 92.71) (end 158.75 86.36) (width 0.25) (layer "B.Cu") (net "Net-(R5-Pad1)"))
 (segment (start 160.315 88.7041) (end 162.56 90.9492) (width 0.25) (layer "F.Cu") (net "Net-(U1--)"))
 (segment (start 144.865 85.3062) (end 147.565 85.3062) (width 0.25) (layer "F.Cu") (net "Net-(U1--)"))
 (segment (start 162.56 90.9492) (end 162.56 91.435) (width 0.25) (layer "F.Cu") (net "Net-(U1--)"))
 (segment (start 143.811 86.36) (end 144.865 85.3062) (width 0.25) (layer "F.Cu") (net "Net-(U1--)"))
 (segment (start 150.963 88.7041) (end 160.315 88.7041) (width 0.25) (layer "F.Cu") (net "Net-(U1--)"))
 (segment (start 143.811 86.36) (end 144.865 85.3062) (width 0.25) (layer "F.Cu") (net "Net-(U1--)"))
 (segment (start 143.51 86.36) (end 139.16 86.36) (width 0.25) (layer "F.Cu") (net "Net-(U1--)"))
 (segment (start 144.865 85.3062) (end 147.565 85.3062) (width 0.25) (layer "F.Cu") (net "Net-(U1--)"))
 (segment (start 162.56 90.9492) (end 162.56 91.435) (width 0.25) (layer "F.Cu") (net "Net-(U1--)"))
 (segment (start 147.565 85.3062) (end 150.963 88.7041) (width 0.25) (layer "F.Cu") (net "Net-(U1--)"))
 (segment (start 143.51 86.36) (end 143.811 86.36) (width 0.25) (layer "F.Cu") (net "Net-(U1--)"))
 (segment (start 147.565 85.3062) (end 150.963 88.7041) (width 0.25) (layer "F.Cu") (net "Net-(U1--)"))
 (segment (start 150.963 88.7041) (end 160.315 88.7041) (width 0.25) (layer "F.Cu") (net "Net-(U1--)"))
 (segment (start 160.315 88.7041) (end 162.56 90.9492) (width 0.25) (layer "F.Cu") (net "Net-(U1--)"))
 (segment (start 178.77 74.4536) (end 184.643 68.58) (width 0.25) (layer "F.Cu") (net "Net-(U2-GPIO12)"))
 (segment (start 178.77 74.4536) (end 184.643 68.58) (width 0.25) (layer "F.Cu") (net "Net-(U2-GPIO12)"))
 (segment (start 185.42 68.58) (end 184.643 68.58) (width 0.25) (layer "F.Cu") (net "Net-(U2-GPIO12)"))
 (segment (start 164.626 74.4536) (end 178.77 74.4536) (width 0.25) (layer "F.Cu") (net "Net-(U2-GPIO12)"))
 (segment (start 184.643 68.58) (end 185.42 68.58) (width 0.25) (layer "F.Cu") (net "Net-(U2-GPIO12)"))
 (via (at 164.626 74.4536) (size 0.8) (drill 0.4) (layers "F.Cu" "B.Cu") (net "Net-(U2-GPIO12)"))
 (segment (start 160.02 80.01) (end 160.02 79.06) (width 0.25) (layer "B.Cu") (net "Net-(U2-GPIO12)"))
 (segment (start 160.02 79.06) (end 164.626 74.4536) (width 0.25) (layer "B.Cu") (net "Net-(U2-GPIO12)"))
 (segment (start 160.02 79.06) (end 164.626 74.4536) (width 0.25) (layer "B.Cu") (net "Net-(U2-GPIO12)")))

